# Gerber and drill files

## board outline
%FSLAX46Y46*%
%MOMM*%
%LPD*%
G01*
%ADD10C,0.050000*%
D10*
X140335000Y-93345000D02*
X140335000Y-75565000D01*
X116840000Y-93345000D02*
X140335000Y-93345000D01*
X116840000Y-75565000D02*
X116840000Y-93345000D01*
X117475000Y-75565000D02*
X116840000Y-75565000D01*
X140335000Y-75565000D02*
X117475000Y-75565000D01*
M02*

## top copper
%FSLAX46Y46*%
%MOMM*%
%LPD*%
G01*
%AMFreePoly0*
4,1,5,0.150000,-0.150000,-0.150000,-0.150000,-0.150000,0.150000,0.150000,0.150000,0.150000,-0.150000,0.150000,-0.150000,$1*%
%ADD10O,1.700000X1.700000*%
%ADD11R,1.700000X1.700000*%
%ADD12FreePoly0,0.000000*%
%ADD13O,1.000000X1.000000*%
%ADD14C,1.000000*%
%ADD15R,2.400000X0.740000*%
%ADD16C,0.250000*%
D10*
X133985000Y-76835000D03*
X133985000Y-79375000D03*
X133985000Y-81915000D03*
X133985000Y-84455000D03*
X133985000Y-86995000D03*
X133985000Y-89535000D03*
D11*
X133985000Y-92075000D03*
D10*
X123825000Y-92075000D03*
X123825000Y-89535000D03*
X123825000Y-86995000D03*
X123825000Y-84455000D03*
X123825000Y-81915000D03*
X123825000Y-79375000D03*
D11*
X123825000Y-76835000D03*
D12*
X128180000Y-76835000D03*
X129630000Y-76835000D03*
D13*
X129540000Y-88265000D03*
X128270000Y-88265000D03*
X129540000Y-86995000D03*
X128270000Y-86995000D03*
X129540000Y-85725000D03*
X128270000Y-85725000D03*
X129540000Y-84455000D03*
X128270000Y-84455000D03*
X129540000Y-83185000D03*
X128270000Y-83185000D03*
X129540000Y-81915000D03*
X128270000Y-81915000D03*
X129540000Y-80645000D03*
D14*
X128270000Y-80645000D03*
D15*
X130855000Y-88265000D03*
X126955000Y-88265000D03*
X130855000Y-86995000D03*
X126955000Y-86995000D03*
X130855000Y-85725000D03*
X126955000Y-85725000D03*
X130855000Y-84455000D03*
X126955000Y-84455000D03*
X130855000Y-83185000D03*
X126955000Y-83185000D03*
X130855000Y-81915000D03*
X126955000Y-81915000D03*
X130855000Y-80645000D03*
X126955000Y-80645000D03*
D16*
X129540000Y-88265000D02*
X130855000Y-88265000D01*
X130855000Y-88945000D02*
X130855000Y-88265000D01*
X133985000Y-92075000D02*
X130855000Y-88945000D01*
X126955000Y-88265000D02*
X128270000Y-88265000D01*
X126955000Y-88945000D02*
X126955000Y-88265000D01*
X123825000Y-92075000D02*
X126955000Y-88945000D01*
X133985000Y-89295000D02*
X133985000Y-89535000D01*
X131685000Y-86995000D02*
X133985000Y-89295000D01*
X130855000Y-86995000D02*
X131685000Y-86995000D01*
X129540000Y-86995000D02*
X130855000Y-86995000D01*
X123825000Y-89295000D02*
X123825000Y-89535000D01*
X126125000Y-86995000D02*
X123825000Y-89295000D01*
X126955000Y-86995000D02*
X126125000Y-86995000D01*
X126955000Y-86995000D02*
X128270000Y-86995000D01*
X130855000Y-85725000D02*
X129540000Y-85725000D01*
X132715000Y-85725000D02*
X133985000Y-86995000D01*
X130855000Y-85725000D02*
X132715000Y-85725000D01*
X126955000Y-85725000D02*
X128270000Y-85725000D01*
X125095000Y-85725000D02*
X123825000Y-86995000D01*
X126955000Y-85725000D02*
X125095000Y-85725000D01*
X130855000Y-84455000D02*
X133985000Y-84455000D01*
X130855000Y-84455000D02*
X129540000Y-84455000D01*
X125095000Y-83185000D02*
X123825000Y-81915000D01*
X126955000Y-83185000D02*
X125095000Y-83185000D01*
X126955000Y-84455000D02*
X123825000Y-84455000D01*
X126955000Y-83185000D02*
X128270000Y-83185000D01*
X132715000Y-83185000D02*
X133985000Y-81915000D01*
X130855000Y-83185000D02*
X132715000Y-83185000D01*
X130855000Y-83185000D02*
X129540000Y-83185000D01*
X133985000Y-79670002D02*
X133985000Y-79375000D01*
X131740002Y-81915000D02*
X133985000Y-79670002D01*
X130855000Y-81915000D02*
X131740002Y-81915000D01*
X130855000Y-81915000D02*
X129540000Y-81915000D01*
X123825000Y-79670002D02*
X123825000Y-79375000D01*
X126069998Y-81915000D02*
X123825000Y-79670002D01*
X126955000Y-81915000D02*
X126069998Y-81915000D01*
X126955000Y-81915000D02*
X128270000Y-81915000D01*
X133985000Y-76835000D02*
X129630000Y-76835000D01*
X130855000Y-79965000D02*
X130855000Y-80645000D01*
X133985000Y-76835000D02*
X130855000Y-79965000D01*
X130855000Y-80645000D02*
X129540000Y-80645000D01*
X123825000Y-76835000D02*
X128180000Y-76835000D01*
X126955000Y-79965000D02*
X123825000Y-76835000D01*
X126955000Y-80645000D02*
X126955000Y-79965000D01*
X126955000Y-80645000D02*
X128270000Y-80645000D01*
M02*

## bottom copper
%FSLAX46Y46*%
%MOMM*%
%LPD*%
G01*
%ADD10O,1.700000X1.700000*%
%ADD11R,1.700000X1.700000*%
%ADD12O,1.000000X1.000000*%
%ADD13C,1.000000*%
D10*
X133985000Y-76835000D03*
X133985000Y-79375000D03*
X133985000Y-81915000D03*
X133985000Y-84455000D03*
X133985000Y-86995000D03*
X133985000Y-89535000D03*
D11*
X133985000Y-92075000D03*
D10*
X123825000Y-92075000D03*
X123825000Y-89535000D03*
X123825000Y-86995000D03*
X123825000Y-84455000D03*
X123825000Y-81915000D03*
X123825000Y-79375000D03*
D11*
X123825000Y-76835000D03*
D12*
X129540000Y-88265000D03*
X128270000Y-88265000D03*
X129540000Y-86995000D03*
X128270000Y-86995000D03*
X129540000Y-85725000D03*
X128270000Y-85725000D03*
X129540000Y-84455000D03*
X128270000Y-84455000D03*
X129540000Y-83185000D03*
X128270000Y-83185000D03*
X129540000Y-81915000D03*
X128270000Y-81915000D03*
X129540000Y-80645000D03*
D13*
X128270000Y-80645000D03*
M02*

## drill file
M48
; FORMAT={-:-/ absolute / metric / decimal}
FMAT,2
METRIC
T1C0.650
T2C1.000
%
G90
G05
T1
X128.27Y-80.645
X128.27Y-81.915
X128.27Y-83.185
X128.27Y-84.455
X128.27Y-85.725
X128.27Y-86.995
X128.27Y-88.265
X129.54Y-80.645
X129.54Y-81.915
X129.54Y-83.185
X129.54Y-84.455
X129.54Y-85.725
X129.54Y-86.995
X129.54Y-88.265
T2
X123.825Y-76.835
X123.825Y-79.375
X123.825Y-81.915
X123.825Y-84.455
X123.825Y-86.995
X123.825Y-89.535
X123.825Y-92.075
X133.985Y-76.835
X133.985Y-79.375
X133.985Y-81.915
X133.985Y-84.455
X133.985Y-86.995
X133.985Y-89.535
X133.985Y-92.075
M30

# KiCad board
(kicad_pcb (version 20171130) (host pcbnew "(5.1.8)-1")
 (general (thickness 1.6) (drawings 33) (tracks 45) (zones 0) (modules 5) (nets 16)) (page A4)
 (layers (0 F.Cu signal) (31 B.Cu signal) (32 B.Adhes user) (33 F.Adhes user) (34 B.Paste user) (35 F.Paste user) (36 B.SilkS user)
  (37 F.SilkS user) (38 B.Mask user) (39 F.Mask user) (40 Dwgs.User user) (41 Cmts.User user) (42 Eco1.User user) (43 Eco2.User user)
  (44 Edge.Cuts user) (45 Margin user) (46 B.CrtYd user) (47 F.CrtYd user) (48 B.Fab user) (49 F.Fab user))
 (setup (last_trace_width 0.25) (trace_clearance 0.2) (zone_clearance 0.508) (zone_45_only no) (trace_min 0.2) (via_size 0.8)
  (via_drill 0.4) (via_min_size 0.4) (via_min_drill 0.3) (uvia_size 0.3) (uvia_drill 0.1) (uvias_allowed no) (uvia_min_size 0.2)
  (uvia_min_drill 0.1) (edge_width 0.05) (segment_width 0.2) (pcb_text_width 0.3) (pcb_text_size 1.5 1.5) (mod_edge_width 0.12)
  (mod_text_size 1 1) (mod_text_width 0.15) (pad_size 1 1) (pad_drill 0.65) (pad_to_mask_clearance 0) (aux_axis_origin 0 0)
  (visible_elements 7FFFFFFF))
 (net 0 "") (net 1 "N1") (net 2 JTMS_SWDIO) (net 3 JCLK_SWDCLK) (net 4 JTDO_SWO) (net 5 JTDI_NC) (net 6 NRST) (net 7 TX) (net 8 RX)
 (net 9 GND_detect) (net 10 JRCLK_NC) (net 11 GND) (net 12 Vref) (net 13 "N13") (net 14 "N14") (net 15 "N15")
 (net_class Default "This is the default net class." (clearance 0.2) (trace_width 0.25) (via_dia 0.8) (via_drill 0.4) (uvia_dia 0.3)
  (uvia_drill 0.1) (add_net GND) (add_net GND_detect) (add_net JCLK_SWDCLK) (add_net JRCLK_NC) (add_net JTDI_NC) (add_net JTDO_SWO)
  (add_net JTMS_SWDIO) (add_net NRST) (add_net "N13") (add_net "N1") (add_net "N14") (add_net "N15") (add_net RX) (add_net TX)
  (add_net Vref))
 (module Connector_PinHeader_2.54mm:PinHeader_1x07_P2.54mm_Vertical (layer B.Cu) (at 133.985 92.075)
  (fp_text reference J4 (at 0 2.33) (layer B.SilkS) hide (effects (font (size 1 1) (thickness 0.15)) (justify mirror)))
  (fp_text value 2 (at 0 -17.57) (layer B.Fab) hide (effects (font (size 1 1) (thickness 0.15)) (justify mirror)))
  (pad 7 thru_hole oval (at 0 -15.24) (size 1.7 1.7) (drill 1) (layers *.Cu *.Mask) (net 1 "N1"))
  (pad 6 thru_hole oval (at 0 -12.7) (size 1.7 1.7) (drill 1) (layers *.Cu *.Mask) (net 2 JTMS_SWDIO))
  (pad 5 thru_hole oval (at 0 -10.16) (size 1.7 1.7) (drill 1) (layers *.Cu *.Mask) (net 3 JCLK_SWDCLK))
  (pad 4 thru_hole oval (at 0 -7.62) (size 1.7 1.7) (drill 1) (layers *.Cu *.Mask) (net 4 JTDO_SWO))
  (pad 3 thru_hole oval (at 0 -5.08) (size 1.7 1.7) (drill 1) (layers *.Cu *.Mask) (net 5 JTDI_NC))
  (pad 2 thru_hole oval (at 0 -2.54) (size 1.7 1.7) (drill 1) (layers *.Cu *.Mask) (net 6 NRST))
  (pad 1 thru_hole rect (at 0 0) (size 1.7 1.7) (drill 1) (layers *.Cu *.Mask) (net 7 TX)))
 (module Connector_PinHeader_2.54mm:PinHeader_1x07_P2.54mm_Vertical (layer B.Cu) (at 123.825 76.835 180)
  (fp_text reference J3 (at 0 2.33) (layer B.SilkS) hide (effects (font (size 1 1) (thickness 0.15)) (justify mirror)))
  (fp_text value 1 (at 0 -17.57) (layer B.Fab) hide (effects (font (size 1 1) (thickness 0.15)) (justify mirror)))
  (pad 7 thru_hole oval (at 0 -15.24 180) (size 1.7 1.7) (drill 1) (layers *.Cu *.Mask) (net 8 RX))
  (pad 6 thru_hole oval (at 0 -12.7 180) (size 1.7 1.7) (drill 1) (layers *.Cu *.Mask) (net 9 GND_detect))
  (pad 5 thru_hole oval (at 0 -10.16 180) (size 1.7 1.7) (drill 1) (layers *.Cu *.Mask) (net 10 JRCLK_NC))
  (pad 4 thru_hole oval (at 0 -7.62 180) (size 1.7 1.7) (drill 1) (layers *.Cu *.Mask) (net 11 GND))
  (pad 3 thru_hole oval (at 0 -5.08 180) (size 1.7 1.7) (drill 1) (layers *.Cu *.Mask) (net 11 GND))
  (pad 2 thru_hole oval (at 0 -2.54 180) (size 1.7 1.7) (drill 1) (layers *.Cu *.Mask) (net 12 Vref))
  (pad 1 thru_hole rect (at 0 0 180) (size 1.7 1.7) (drill 1) (layers *.Cu *.Mask) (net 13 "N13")))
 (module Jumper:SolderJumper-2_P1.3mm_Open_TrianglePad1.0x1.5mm (layer F.Cu) (at 128.905 76.835)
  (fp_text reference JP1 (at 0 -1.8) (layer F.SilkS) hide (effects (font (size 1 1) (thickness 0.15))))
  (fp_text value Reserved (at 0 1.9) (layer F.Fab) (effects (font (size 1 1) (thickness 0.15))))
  (pad 1 smd custom (at -0.725 0) (size 0.3 0.3) (layers F.Cu F.Mask) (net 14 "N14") (zone_connect 2)
   (options (clearance outline) (anchor rect)) (primitives))
  (pad 2 smd custom (at 0.725 0) (size 0.3 0.3) (layers F.Cu F.Mask) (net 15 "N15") (zone_connect 2)
   (options (clearance outline) (anchor rect)) (primitives)))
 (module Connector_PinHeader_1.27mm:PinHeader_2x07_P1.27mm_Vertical (layer F.Cu) (at 128.27 80.645)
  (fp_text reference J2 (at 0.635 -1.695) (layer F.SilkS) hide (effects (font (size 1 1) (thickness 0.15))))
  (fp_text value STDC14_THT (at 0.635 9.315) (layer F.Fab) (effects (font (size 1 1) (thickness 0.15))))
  (pad 14 thru_hole oval (at 1.27 7.62) (size 1 1) (drill 0.65) (layers *.Cu *.Mask) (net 7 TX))
  (pad 13 thru_hole oval (at 0 7.62) (size 1 1) (drill 0.65) (layers *.Cu *.Mask) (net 8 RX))
  (pad 12 thru_hole oval (at 1.27 6.35) (size 1 1) (drill 0.65) (layers *.Cu *.Mask) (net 6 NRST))
  (pad 11 thru_hole oval (at 0 6.35) (size 1 1) (drill 0.65) (layers *.Cu *.Mask) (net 9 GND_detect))
  (pad 10 thru_hole oval (at 1.27 5.08) (size 1 1) (drill 0.65) (layers *.Cu *.Mask) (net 5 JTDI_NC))
  (pad 9 thru_hole oval (at 0 5.08) (size 1 1) (drill 0.65) (layers *.Cu *.Mask) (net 10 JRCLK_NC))
  (pad 8 thru_hole oval (at 1.27 3.81) (size 1 1) (drill 0.65) (layers *.Cu *.Mask) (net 4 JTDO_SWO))
  (pad 7 thru_hole oval (at 0 3.81) (size 1 1) (drill 0.65) (layers *.Cu *.Mask) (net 11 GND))
  (pad 6 thru_hole oval (at 1.27 2.54) (size 1 1) (drill 0.65) (layers *.Cu *.Mask) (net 3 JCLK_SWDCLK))
  (pad 5 thru_hole oval (at 0 2.54) (size 1 1) (drill 0.65) (layers *.Cu *.Mask) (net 11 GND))
  (pad 4 thru_hole oval (at 1.27 1.27) (size 1 1) (drill 0.65) (layers *.Cu *.Mask) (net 2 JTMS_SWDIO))
  (pad 3 thru_hole oval (at 0 1.27) (size 1 1) (drill 0.65) (layers *.Cu *.Mask) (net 12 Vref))
  (pad 2 thru_hole oval (at 1.27 0) (size 1 1) (drill 0.65) (layers *.Cu *.Mask) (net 1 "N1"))
  (pad 1 thru_hole circle (at 0 0) (size 1 1) (drill 0.65) (layers *.Cu *.Mask) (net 13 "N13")))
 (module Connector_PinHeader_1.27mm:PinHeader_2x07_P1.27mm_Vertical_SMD (layer F.Cu) (at 128.905 84.455)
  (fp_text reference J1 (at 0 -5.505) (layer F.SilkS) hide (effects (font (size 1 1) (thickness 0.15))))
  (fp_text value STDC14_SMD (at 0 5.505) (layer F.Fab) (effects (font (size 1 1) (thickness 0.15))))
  (pad 14 smd rect (at 1.95 3.81) (size 2.4 0.74) (layers F.Cu F.Paste F.Mask) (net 7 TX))
  (pad 13 smd rect (at -1.95 3.81) (size 2.4 0.74) (layers F.Cu F.Paste F.Mask) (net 8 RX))
  (pad 12 smd rect (at 1.95 2.54) (size 2.4 0.74) (layers F.Cu F.Paste F.Mask) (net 6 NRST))
  (pad 11 smd rect (at -1.95 2.54) (size 2.4 0.74) (layers F.Cu F.Paste F.Mask) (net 9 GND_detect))
  (pad 10 smd rect (at 1.95 1.27) (size 2.4 0.74) (layers F.Cu F.Paste F.Mask) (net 5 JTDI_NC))
  (pad 9 smd rect (at -1.95 1.27) (size 2.4 0.74) (layers F.Cu F.Paste F.Mask) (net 10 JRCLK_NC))
  (pad 8 smd rect (at 1.95 0) (size 2.4 0.74) (layers F.Cu F.Paste F.Mask) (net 4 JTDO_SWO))
  (pad 7 smd rect (at -1.95 0) (size 2.4 0.74) (layers F.Cu F.Paste F.Mask) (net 11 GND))
  (pad 6 smd rect (at 1.95 -1.27) (size 2.4 0.74) (layers F.Cu F.Paste F.Mask) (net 3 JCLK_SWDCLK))
  (pad 5 smd rect (at -1.95 -1.27) (size 2.4 0.74) (layers F.Cu F.Paste F.Mask) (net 11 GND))
  (pad 4 smd rect (at 1.95 -2.54) (size 2.4 0.74) (layers F.Cu F.Paste F.Mask) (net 2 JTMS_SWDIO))
  (pad 3 smd rect (at -1.95 -2.54) (size 2.4 0.74) (layers F.Cu F.Paste F.Mask) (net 12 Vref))
  (pad 2 smd rect (at 1.95 -3.81) (size 2.4 0.74) (layers F.Cu F.Paste F.Mask) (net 1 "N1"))
  (pad 1 smd rect (at -1.95 -3.81) (size 2.4 0.74) (layers F.Cu F.Paste F.Mask) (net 13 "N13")))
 (gr_line (start 140.335 93.345) (end 140.335 75.565) (layer Edge.Cuts) (width 0.05))
 (gr_line (start 116.84 93.345) (end 140.335 93.345) (layer Edge.Cuts) (width 0.05))
 (gr_line (start 116.84 75.565) (end 116.84 93.345) (layer Edge.Cuts) (width 0.05))
 (gr_line (start 117.475 75.565) (end 116.84 75.565) (layer Edge.Cuts) (width 0.05))
 (gr_line (start 140.335 75.565) (end 117.475 75.565) (layer Edge.Cuts) (width 0.05))
 (segment (start 129.54 88.265) (end 130.855 88.265) (width 0.25) (layer F.Cu) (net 7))
 (segment (start 130.855 88.945) (end 130.855 88.265) (width 0.25) (layer F.Cu) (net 7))
 (segment (start 133.985 92.075) (end 130.855 88.945) (width 0.25) (layer F.Cu) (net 7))
 (segment (start 126.955 88.265) (end 128.27 88.265) (width 0.25) (layer F.Cu) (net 8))
 (segment (start 126.955 88.945) (end 126.955 88.265) (width 0.25) (layer F.Cu) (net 8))
 (segment (start 123.825 92.075) (end 126.955 88.945) (width 0.25) (layer F.Cu) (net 8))
 (segment (start 133.985 89.295) (end 133.985 89.535) (width 0.25) (layer F.Cu) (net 6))
 (segment (start 131.685 86.995) (end 133.985 89.295) (width 0.25) (layer F.Cu) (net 6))
 (segment (start 130.855 86.995) (end 131.685 86.995) (width 0.25) (layer F.Cu) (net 6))
 (segment (start 129.54 86.995) (end 130.855 86.995) (width 0.25) (layer F.Cu) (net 6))
 (segment (start 123.825 89.295) (end 123.825 89.535) (width 0.25) (layer F.Cu) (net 9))
 (segment (start 126.125 86.995) (end 123.825 89.295) (width 0.25) (layer F.Cu) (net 9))
 (segment (start 126.955 86.995) (end 126.125 86.995) (width 0.25) (layer F.Cu) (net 9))
 (segment (start 126.955 86.995) (end 128.27 86.995) (width 0.25) (layer F.Cu) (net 9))
 (segment (start 130.855 85.725) (end 129.54 85.725) (width 0.25) (layer F.Cu) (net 5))
 (segment (start 132.715 85.725) (end 133.985 86.995) (width 0.25) (layer F.Cu) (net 5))
 (segment (start 130.855 85.725) (end 132.715 85.725) (width 0.25) (layer F.Cu) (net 5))
 (segment (start 126.955 85.725) (end 128.27 85.725) (width 0.25) (layer F.Cu) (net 10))
 (segment (start 125.095 85.725) (end 123.825 86.995) (width 0.25) (layer F.Cu) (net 10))
 (segment (start 126.955 85.725) (end 125.095 85.725) (width 0.25) (layer F.Cu) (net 10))
 (segment (start 130.855 84.455) (end 133.985 84.455) (width 0.25) (layer F.Cu) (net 4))
 (segment (start 130.855 84.455) (end 129.54 84.455) (width 0.25) (layer F.Cu) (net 4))
 (segment (start 125.095 83.185) (end 123.825 81.915) (width 0.25) (layer F.Cu) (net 11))
 (segment (start 126.955 83.185) (end 125.095 83.185) (width 0.25) (layer F.Cu) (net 11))
 (segment (start 126.955 84.455) (end 123.825 84.455) (width 0.25) (layer F.Cu) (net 11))
 (segment (start 126.955 83.185) (end 128.27 83.185) (width 0.25) (layer F.Cu) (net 11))
 (segment (start 132.715 83.185) (end 133.985 81.915) (width 0.25) (layer F.Cu) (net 3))
 (segment (start 130.855 83.185) (end 132.715 83.185) (width 0.25) (layer F.Cu) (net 3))
 (segment (start 130.855 83.185) (end 129.54 83.185) (width 0.25) (layer F.Cu) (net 3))
 (segment (start 133.985 79.670002) (end 133.985 79.375) (width 0.25) (layer F.Cu) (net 2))
 (segment (start 131.740002 81.915) (end 133.985 79.670002) (width 0.25) (layer F.Cu) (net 2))
 (segment (start 130.855 81.915) (end 131.740002 81.915) (width 0.25) (layer F.Cu) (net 2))
 (segment (start 130.855 81.915) (end 129.54 81.915) (width 0.25) (layer F.Cu) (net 2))
 (segment (start 123.825 79.670002) (end 123.825 79.375) (width 0.25) (layer F.Cu) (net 12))
 (segment (start 126.069998 81.915) (end 123.825 79.670002) (width 0.25) (layer F.Cu) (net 12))
 (segment (start 126.955 81.915) (end 126.069998 81.915) (width 0.25) (layer F.Cu) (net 12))
 (segment (start 126.955 81.915) (end 128.27 81.915) (width 0.25) (layer F.Cu) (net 12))
 (segment (start 133.985 76.835) (end 129.63 76.835) (width 0.25) (layer F.Cu) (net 1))
 (segment (start 130.855 79.965) (end 130.855 80.645) (width 0.25) (layer F.Cu) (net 1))
 (segment (start 133.985 76.835) (end 130.855 79.965) (width 0.25) (layer F.Cu) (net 1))
 (segment (start 130.855 80.645) (end 129.54 80.645) (width 0.25) (layer F.Cu) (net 1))
 (segment (start 123.825 76.835) (end 128.18 76.835) (width 0.25) (layer F.Cu) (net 13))
 (segment (start 126.955 79.965) (end 123.825 76.835) (width 0.25) (layer F.Cu) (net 13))
 (segment (start 126.955 80.645) (end 126.955 79.965) (width 0.25) (layer F.Cu) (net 13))
 (segment (start 126.955 80.645) (end 128.27 80.645) (width 0.25) (layer F.Cu) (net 13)))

